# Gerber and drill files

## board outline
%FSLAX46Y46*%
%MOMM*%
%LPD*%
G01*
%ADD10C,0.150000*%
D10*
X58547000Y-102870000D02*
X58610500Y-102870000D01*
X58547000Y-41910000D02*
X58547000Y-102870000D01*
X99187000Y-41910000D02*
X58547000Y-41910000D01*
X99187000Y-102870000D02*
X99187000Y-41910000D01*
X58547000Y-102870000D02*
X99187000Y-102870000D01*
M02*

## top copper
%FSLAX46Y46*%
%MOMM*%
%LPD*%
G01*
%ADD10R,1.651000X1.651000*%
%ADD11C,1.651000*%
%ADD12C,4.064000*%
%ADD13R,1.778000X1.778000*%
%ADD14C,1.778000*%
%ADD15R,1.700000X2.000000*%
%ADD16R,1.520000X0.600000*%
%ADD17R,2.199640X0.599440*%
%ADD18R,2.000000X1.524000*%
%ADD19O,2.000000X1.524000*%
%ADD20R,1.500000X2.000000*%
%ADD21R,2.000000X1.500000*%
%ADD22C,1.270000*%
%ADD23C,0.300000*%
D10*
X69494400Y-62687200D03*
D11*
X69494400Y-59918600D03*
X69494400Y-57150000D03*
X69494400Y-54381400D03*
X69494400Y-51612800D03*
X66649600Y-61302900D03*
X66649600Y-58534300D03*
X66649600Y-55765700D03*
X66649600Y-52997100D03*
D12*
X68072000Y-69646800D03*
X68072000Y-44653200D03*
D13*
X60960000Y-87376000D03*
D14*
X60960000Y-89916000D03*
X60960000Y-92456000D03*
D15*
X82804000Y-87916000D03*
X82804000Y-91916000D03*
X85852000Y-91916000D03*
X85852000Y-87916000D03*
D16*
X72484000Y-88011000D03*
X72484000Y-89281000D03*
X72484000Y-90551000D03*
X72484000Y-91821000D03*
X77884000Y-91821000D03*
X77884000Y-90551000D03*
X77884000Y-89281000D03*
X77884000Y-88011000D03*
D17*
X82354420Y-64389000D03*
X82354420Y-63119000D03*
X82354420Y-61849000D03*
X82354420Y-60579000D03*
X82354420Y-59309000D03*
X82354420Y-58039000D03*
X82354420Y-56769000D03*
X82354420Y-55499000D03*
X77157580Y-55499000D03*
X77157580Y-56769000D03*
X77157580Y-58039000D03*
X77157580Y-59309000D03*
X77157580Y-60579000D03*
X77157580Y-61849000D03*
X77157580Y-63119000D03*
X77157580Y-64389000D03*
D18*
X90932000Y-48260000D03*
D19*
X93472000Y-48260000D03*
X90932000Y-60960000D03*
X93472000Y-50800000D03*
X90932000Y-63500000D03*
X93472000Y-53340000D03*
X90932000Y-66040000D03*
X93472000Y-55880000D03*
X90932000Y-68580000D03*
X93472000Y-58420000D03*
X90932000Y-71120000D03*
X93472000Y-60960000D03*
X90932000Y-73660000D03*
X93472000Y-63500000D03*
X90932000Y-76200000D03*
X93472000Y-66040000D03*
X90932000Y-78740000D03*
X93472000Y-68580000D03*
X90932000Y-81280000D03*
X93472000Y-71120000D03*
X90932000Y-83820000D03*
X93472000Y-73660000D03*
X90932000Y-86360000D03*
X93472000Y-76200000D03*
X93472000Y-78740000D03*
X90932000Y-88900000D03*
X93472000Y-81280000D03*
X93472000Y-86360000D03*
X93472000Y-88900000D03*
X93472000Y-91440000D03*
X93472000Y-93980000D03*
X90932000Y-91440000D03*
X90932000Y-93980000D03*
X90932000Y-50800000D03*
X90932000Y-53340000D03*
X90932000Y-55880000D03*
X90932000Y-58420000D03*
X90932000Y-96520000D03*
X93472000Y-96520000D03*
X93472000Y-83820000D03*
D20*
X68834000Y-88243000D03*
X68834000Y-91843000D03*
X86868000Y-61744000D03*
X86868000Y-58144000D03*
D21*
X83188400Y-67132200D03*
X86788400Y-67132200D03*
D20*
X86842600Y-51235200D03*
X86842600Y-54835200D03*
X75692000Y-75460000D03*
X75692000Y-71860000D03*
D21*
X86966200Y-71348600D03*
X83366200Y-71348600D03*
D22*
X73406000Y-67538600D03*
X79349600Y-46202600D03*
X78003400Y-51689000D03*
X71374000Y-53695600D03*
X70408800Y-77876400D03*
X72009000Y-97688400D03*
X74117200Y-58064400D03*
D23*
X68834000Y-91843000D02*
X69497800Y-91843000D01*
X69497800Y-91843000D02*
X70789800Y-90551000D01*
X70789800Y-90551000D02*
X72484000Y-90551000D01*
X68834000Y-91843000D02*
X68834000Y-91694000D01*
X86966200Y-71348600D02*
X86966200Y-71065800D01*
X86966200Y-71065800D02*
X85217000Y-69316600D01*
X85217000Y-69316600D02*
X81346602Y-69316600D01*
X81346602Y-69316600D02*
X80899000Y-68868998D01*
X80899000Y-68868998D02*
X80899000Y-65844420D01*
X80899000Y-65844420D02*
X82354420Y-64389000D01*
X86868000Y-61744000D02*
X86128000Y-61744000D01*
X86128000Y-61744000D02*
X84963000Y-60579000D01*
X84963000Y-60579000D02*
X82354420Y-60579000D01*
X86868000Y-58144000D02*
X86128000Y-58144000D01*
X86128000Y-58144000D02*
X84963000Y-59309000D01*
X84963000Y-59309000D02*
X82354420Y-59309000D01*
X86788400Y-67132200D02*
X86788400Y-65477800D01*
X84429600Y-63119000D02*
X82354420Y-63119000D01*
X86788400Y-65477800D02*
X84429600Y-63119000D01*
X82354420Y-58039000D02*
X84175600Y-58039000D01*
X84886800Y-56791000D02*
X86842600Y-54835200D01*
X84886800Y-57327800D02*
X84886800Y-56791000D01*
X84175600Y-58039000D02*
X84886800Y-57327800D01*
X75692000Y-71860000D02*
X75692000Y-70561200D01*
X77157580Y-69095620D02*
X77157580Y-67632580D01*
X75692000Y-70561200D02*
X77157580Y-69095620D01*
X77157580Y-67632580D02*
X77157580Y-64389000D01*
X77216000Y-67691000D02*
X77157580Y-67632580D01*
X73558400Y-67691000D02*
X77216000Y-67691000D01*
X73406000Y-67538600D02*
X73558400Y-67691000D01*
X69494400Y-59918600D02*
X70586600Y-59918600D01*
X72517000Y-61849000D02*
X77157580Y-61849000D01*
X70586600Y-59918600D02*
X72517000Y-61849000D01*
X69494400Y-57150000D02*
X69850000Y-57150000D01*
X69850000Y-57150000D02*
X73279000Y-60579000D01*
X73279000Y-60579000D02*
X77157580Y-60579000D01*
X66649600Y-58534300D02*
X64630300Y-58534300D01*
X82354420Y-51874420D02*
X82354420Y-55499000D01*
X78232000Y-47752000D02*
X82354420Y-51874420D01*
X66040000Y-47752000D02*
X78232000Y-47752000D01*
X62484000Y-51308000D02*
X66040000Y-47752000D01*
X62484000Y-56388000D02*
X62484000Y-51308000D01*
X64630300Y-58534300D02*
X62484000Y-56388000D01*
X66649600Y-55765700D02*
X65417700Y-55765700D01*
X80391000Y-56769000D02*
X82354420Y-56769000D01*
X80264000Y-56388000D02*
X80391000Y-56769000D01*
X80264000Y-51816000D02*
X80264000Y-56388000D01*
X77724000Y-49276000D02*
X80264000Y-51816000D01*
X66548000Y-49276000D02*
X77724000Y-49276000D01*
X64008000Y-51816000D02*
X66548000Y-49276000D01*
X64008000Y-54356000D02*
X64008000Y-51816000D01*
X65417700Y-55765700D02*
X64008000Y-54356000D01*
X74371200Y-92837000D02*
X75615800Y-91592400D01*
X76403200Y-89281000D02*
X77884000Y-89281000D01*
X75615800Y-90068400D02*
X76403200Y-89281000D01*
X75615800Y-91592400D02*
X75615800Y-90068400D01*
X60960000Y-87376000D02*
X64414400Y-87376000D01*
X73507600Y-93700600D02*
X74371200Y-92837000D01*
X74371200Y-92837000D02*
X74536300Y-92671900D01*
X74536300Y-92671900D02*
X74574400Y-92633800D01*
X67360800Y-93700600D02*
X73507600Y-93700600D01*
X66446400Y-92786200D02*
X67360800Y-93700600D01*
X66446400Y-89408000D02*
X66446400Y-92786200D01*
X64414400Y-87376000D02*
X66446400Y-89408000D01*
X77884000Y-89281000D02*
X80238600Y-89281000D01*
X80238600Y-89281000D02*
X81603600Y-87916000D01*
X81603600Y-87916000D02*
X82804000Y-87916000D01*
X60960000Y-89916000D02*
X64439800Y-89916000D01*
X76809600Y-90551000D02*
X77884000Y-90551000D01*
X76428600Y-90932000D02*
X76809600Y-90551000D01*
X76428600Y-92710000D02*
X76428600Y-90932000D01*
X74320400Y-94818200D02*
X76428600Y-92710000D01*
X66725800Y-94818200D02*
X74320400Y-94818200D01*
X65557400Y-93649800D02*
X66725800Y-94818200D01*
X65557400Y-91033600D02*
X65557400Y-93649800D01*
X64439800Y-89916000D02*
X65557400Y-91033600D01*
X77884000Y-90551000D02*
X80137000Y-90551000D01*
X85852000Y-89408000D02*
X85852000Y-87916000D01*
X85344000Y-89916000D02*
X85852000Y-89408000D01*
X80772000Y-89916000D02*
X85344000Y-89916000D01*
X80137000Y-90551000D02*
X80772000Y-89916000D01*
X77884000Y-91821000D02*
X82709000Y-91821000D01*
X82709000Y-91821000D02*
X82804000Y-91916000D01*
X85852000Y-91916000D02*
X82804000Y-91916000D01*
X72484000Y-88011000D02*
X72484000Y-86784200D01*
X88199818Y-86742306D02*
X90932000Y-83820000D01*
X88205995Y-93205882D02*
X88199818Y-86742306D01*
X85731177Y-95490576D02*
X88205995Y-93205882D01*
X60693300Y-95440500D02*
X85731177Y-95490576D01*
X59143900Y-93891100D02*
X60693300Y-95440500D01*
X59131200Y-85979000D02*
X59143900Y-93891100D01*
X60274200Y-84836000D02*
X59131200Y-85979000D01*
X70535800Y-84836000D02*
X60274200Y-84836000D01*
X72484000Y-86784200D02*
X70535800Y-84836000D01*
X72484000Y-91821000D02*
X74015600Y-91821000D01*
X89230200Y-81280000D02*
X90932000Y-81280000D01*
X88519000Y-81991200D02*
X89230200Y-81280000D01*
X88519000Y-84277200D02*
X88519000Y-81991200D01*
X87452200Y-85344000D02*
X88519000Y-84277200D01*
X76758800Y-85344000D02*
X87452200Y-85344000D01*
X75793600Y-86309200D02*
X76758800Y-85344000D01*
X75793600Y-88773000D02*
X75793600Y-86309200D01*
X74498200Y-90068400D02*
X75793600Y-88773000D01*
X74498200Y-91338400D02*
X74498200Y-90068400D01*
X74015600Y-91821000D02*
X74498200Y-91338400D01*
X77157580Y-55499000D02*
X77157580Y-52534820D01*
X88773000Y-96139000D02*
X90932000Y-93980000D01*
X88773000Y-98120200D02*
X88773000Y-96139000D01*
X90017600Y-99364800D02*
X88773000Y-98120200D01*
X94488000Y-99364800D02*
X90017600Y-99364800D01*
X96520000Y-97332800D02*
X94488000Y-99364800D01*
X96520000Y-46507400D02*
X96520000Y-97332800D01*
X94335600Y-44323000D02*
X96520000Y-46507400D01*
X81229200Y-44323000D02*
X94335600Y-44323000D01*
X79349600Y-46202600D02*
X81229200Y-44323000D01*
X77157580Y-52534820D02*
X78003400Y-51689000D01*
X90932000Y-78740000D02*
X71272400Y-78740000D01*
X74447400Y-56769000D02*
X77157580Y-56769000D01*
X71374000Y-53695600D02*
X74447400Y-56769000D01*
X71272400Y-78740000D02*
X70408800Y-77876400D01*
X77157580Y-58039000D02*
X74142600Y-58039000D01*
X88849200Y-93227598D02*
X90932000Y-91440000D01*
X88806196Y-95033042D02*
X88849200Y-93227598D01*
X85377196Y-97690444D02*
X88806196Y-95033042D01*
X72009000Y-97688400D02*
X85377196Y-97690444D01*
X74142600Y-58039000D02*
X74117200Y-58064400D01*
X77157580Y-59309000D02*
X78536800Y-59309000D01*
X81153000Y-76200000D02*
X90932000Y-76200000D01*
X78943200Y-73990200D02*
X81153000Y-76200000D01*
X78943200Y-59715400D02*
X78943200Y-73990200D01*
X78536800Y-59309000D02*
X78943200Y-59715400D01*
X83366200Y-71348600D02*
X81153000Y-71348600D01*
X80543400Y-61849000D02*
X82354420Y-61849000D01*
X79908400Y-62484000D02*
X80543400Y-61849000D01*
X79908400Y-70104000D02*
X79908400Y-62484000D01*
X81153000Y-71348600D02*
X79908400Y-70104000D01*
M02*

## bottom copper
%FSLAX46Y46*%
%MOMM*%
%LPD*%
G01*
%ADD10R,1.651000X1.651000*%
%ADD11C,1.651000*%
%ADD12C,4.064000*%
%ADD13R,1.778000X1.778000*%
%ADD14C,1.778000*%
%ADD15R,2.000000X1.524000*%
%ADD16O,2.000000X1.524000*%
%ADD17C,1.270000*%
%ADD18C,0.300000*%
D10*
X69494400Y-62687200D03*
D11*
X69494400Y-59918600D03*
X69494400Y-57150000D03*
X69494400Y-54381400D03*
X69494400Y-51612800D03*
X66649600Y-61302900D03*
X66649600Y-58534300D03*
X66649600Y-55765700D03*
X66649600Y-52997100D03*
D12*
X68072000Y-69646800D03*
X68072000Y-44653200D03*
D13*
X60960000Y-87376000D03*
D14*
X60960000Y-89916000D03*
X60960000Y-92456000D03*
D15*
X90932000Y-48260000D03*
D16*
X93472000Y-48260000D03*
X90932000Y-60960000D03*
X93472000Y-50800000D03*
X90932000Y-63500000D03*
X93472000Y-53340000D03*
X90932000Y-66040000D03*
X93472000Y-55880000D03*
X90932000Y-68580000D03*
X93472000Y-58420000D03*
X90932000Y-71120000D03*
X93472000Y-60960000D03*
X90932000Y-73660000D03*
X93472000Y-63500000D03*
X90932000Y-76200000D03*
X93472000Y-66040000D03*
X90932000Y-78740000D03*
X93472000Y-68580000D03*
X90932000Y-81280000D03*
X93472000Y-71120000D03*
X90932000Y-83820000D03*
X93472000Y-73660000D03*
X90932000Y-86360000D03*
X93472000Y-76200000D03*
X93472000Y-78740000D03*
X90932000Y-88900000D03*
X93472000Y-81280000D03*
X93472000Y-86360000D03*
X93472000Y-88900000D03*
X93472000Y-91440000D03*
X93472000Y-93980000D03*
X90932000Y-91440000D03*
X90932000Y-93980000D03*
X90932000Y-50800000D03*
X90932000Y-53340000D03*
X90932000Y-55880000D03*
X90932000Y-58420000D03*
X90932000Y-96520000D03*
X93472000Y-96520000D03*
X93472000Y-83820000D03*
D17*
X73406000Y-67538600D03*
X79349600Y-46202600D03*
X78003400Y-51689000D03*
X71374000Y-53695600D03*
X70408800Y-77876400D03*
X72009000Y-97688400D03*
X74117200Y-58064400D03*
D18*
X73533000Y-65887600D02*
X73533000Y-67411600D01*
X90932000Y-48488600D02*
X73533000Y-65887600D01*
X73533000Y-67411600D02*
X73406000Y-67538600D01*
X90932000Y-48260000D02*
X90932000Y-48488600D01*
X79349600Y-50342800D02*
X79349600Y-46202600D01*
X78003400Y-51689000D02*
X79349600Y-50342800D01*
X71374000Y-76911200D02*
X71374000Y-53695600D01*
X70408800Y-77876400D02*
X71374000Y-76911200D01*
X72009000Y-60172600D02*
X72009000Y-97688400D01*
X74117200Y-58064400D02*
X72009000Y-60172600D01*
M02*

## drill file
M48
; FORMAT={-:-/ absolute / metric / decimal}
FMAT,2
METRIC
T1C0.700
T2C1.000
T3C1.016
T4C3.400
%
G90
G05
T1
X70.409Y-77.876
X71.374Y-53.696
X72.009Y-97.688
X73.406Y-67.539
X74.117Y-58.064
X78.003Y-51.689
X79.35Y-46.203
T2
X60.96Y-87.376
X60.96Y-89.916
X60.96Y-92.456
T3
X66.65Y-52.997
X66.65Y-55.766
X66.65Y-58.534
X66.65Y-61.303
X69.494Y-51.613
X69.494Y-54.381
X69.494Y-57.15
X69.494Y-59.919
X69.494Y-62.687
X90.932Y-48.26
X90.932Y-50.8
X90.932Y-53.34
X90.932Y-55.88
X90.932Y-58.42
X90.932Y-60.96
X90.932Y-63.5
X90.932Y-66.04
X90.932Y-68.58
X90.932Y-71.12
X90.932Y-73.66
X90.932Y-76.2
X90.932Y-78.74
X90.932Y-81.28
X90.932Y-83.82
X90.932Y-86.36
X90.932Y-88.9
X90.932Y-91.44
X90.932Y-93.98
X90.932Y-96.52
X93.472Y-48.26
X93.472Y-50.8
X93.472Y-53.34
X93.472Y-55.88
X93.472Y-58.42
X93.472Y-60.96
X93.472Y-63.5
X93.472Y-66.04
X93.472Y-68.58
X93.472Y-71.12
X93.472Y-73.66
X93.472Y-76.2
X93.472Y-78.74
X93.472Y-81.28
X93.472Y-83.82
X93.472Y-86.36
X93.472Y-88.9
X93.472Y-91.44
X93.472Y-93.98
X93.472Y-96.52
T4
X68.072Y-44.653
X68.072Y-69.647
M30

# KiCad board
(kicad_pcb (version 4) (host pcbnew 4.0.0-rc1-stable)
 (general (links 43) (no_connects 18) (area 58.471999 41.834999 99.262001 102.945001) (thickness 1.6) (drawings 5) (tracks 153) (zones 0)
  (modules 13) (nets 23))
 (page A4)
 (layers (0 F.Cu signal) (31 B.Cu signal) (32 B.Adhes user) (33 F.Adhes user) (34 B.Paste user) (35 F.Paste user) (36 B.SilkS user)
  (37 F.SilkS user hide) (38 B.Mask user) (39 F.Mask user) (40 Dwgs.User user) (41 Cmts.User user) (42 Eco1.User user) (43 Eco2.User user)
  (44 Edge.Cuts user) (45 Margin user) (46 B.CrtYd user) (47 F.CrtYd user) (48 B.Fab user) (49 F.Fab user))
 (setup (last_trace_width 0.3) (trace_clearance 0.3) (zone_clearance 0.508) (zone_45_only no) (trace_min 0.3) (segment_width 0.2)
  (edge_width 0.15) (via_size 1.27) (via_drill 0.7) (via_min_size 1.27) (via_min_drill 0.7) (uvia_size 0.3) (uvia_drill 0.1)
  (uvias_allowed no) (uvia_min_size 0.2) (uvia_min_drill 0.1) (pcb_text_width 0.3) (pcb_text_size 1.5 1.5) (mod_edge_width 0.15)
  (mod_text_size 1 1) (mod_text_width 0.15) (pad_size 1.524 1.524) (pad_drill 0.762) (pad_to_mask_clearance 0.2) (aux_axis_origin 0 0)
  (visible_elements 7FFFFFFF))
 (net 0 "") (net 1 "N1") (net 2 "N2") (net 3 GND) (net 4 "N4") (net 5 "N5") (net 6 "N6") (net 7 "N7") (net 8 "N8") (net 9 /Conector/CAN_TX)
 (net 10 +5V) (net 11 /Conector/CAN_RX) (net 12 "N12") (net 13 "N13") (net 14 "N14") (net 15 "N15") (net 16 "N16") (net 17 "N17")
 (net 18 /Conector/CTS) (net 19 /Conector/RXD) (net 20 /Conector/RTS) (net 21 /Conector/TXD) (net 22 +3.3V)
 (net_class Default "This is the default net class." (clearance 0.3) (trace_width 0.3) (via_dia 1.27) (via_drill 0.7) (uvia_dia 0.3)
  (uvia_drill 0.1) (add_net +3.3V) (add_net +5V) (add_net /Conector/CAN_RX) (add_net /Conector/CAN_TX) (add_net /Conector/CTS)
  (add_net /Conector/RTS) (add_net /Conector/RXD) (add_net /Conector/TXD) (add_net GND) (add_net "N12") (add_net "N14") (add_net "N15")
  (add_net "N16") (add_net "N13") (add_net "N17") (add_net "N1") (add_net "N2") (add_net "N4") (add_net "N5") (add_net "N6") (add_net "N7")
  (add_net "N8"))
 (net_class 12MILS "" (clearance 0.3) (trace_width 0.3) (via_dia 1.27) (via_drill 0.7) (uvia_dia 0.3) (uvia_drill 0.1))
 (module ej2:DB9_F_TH (layer F.Cu) (at 68.072 57.15 90)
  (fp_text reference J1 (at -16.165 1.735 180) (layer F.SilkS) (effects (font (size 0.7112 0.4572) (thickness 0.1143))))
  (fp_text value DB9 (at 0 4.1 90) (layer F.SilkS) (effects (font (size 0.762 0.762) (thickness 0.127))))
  (pad 1 thru_hole rect (at -5.5372 1.4224 90) (size 1.651 1.651) (drill 1.016) (layers *.Cu *.Mask))
  (pad 2 thru_hole circle (at -2.7686 1.4224 90) (size 1.651 1.651) (drill 1.016) (layers *.Cu *.Mask) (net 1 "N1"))
  (pad 3 thru_hole circle (at 0 1.4224 90) (size 1.651 1.651) (drill 1.016) (layers *.Cu *.Mask) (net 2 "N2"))
  (pad 4 thru_hole circle (at 2.7686 1.4224 90) (size 1.651 1.651) (drill 1.016) (layers *.Cu *.Mask))
  (pad 5 thru_hole circle (at 5.5372 1.4224 90) (size 1.651 1.651) (drill 1.016) (layers *.Cu *.Mask) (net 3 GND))
  (pad 6 thru_hole circle (at -4.1529 -1.4224 90) (size 1.651 1.651) (drill 1.016) (layers *.Cu *.Mask))
  (pad 7 thru_hole circle (at -1.3843 -1.4224 90) (size 1.651 1.651) (drill 1.016) (layers *.Cu *.Mask) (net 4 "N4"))
  (pad 8 thru_hole circle (at 1.3843 -1.4224 90) (size 1.651 1.651) (drill 1.016) (layers *.Cu *.Mask) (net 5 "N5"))
  (pad 9 thru_hole circle (at 4.1529 -1.4224 90) (size 1.651 1.651) (drill 1.016) (layers *.Cu *.Mask))
  (pad 10 thru_hole circle (at -12.4968 0 90) (size 4.064 4.064) (drill 3.4) (layers *.Cu *.Mask))
  (pad 11 thru_hole circle (at 12.4968 0 90) (size 4.064 4.064) (drill 3.4) (layers *.Cu *.Mask)))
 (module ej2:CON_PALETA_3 (layer F.Cu) (at 60.96 89.916 270)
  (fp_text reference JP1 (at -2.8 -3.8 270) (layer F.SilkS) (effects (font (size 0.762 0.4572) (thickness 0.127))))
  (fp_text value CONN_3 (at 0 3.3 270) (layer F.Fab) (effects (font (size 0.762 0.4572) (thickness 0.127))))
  (pad 1 thru_hole rect (at -2.54 0 270) (size 1.778 1.778) (drill 1) (layers *.Cu *.Mask) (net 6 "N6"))
  (pad 2 thru_hole circle (at 0 0 270) (size 1.778 1.778) (drill 1) (layers *.Cu *.Mask) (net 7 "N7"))
  (pad 3 thru_hole circle (at 2.54 0 270) (size 1.778 1.778) (drill 1) (layers *.Cu *.Mask)))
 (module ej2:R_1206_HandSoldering (layer F.Cu) (at 82.804 89.916 270)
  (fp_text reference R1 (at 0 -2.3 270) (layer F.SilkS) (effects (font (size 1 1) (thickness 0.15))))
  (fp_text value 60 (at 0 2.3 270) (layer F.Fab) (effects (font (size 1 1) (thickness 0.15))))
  (pad 1 smd rect (at -2 0 270) (size 2 1.7) (layers F.Cu F.Paste F.Mask) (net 6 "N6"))
  (pad 2 smd rect (at 2 0 270) (size 2 1.7) (layers F.Cu F.Paste F.Mask) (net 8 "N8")))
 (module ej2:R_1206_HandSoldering (layer F.Cu) (at 85.852 89.916 90)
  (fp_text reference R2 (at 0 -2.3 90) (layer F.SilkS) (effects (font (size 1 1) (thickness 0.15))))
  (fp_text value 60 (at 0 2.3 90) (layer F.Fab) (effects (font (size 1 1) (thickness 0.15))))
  (pad 1 smd rect (at -2 0 90) (size 2 1.7) (layers F.Cu F.Paste F.Mask) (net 8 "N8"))
  (pad 2 smd rect (at 2 0 90) (size 2 1.7) (layers F.Cu F.Paste F.Mask) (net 7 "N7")))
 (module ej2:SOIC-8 (layer F.Cu) (at 75.184 89.916)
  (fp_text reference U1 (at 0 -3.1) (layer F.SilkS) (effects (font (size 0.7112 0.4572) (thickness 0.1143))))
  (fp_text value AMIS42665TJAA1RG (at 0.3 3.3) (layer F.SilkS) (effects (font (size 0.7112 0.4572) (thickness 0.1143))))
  (pad 1 smd rect (at -2.7 -1.905 270) (size 0.6 1.52) (layers F.Cu F.Paste F.Mask) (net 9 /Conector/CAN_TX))
  (pad 2 smd rect (at -2.7 -0.635 270) (size 0.6 1.52) (layers F.Cu F.Paste F.Mask) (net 3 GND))
  (pad 3 smd rect (at -2.7 0.635 270) (size 0.6 1.52) (layers F.Cu F.Paste F.Mask) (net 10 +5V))
  (pad 4 smd rect (at -2.7 1.905 270) (size 0.6 1.52) (layers F.Cu F.Paste F.Mask) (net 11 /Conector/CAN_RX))
  (pad 5 smd rect (at 2.7 1.905 270) (size 0.6 1.52) (layers F.Cu F.Paste F.Mask) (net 8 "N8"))
  (pad 6 smd rect (at 2.7 0.635 270) (size 0.6 1.52) (layers F.Cu F.Paste F.Mask) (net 7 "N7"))
  (pad 7 smd rect (at 2.7 -0.635 270) (size 0.6 1.52) (layers F.Cu F.Paste F.Mask) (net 6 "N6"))
  (pad 8 smd rect (at 2.7 -1.905 270) (size 0.6 1.52) (layers F.Cu F.Paste F.Mask) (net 3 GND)))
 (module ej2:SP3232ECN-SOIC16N (layer F.Cu) (at 79.756 59.944 90)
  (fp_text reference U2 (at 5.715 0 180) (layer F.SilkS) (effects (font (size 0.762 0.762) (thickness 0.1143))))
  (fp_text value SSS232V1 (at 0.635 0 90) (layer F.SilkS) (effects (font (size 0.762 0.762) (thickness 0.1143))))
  (pad 1 smd rect (at -4.445 2.59842 90) (size 0.59944 2.19964) (layers F.Cu F.Paste F.Mask) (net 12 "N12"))
  (pad 2 smd rect (at -3.175 2.59842 90) (size 0.59944 2.19964) (layers F.Cu F.Paste F.Mask) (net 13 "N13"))
  (pad 3 smd rect (at -1.905 2.59842 90) (size 0.59944 2.19964) (layers F.Cu F.Paste F.Mask) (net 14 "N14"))
  (pad 4 smd rect (at -0.635 2.59842 90) (size 0.59944 2.19964) (layers F.Cu F.Paste F.Mask) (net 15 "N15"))
  (pad 5 smd rect (at 0.635 2.59842 90) (size 0.59944 2.19964) (layers F.Cu F.Paste F.Mask) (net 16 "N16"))
  (pad 6 smd rect (at 1.905 2.59842 90) (size 0.59944 2.19964) (layers F.Cu F.Paste F.Mask) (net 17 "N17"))
  (pad 7 smd rect (at 3.175 2.59842 90) (size 0.59944 2.19964) (layers F.Cu F.Paste F.Mask) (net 5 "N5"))
  (pad 8 smd rect (at 4.445 2.59842 90) (size 0.59944 2.19964) (layers F.Cu F.Paste F.Mask) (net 4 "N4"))
  (pad 9 smd rect (at 4.445 -2.59842 90) (size 0.59944 2.19964) (layers F.Cu F.Paste F.Mask) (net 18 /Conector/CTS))
  (pad 10 smd rect (at 3.175 -2.59842 90) (size 0.59944 2.19964) (layers F.Cu F.Paste F.Mask) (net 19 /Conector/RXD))
  (pad 11 smd rect (at 1.905 -2.59842 90) (size 0.59944 2.19964) (layers F.Cu F.Paste F.Mask) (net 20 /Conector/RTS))
  (pad 12 smd rect (at 0.635 -2.59842 90) (size 0.59944 2.19964) (layers F.Cu F.Paste F.Mask) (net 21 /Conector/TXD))
  (pad 13 smd rect (at -0.635 -2.59842 90) (size 0.59944 2.19964) (layers F.Cu F.Paste F.Mask) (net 2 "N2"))
  (pad 14 smd rect (at -1.905 -2.59842 90) (size 0.59944 2.19964) (layers F.Cu F.Paste F.Mask) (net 1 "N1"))
  (pad 15 smd rect (at -3.175 -2.59842 90) (size 0.59944 2.19964) (layers F.Cu F.Paste F.Mask) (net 3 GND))
  (pad 16 smd rect (at -4.445 -2.59842 90) (size 0.59944 2.19964) (layers F.Cu F.Paste F.Mask) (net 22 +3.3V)))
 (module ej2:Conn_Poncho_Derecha (layer F.Cu) (at 90.932 48.26)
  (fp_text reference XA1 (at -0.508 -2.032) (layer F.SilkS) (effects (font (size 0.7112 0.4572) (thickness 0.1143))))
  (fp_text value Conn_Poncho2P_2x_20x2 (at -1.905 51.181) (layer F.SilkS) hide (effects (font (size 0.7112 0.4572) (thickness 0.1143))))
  (pad 1 thru_hole rect (at 0 0 270) (size 1.524 2) (drill 1.016) (layers *.Cu *.Mask) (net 22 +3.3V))
  (pad 2 thru_hole oval (at 2.54 0 270) (size 1.524 2) (drill 1.016) (layers *.Cu *.Mask) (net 10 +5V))
  (pad 11 thru_hole oval (at 0 12.7 270) (size 1.524 2) (drill 1.016) (layers *.Cu *.Mask))
  (pad 4 thru_hole oval (at 2.54 2.54 270) (size 1.524 2) (drill 1.016) (layers *.Cu *.Mask) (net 3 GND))
  (pad 13 thru_hole oval (at 0 15.24 270) (size 1.524 2) (drill 1.016) (layers *.Cu *.Mask))
  (pad 6 thru_hole oval (at 2.54 5.08 270) (size 1.524 2) (drill 1.016) (layers *.Cu *.Mask))
  (pad 15 thru_hole oval (at 0 17.78 270) (size 1.524 2) (drill 1.016) (layers *.Cu *.Mask))
  (pad 8 thru_hole oval (at 2.54 7.62 270) (size 1.524 2) (drill 1.016) (layers *.Cu *.Mask))
  (pad 17 thru_hole oval (at 0 20.32 270) (size 1.524 2) (drill 1.016) (layers *.Cu *.Mask))
  (pad 10 thru_hole oval (at 2.54 10.16 270) (size 1.524 2) (drill 1.016) (layers *.Cu *.Mask))
  (pad 19 thru_hole oval (at 0 22.86 270) (size 1.524 2) (drill 1.016) (layers *.Cu *.Mask))
  (pad 12 thru_hole oval (at 2.54 12.7 270) (size 1.524 2) (drill 1.016) (layers *.Cu *.Mask))
  (pad 21 thru_hole oval (at 0 25.4 270) (size 1.524 2) (drill 1.016) (layers *.Cu *.Mask))
  (pad 14 thru_hole oval (at 2.54 15.24 270) (size 1.524 2) (drill 1.016) (layers *.Cu *.Mask))
  (pad 23 thru_hole oval (at 0 27.94 270) (size 1.524 2) (drill 1.016) (layers *.Cu *.Mask) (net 21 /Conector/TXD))
  (pad 16 thru_hole oval (at 2.54 17.78 270) (size 1.524 2) (drill 1.016) (layers *.Cu *.Mask))
  (pad 25 thru_hole oval (at 0 30.48 270) (size 1.524 2) (drill 1.016) (layers *.Cu *.Mask) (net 19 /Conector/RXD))
  (pad 18 thru_hole oval (at 2.54 20.32 270) (size 1.524 2) (drill 1.016) (layers *.Cu *.Mask))
  (pad 27 thru_hole oval (at 0 33.02 270) (size 1.524 2) (drill 1.016) (layers *.Cu *.Mask) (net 11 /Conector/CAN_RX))
  (pad 20 thru_hole oval (at 2.54 22.86 270) (size 1.524 2) (drill 1.016) (layers *.Cu *.Mask) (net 3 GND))
  (pad 29 thru_hole oval (at 0 35.56 270) (size 1.524 2) (drill 1.016) (layers *.Cu *.Mask) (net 9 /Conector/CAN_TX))
  (pad 22 thru_hole oval (at 2.54 25.4 270) (size 1.524 2) (drill 1.016) (layers *.Cu *.Mask) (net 3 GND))
  (pad 31 thru_hole oval (at 0 38.1 270) (size 1.524 2) (drill 1.016) (layers *.Cu *.Mask))
  (pad 24 thru_hole oval (at 2.54 27.94 270) (size 1.524 2) (drill 1.016) (layers *.Cu *.Mask) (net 3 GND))
  (pad 26 thru_hole oval (at 2.54 30.48 270) (size 1.524 2) (drill 1.016) (layers *.Cu *.Mask) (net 3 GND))
  (pad 33 thru_hole oval (at 0 40.64 270) (size 1.524 2) (drill 1.016) (layers *.Cu *.Mask))
  (pad 28 thru_hole oval (at 2.54 33.02 270) (size 1.524 2) (drill 1.016) (layers *.Cu *.Mask) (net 3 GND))
  (pad 32 thru_hole oval (at 2.54 38.1 270) (size 1.524 2) (drill 1.016) (layers *.Cu *.Mask) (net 3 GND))
  (pad 34 thru_hole oval (at 2.54 40.64 270) (size 1.524 2) (drill 1.016) (layers *.Cu *.Mask))
  (pad 36 thru_hole oval (at 2.54 43.18 270) (size 1.524 2) (drill 1.016) (layers *.Cu *.Mask))
  (pad 38 thru_hole oval (at 2.54 45.72 270) (size 1.524 2) (drill 1.016) (layers *.Cu *.Mask) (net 3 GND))
  (pad 35 thru_hole oval (at 0 43.18 270) (size 1.524 2) (drill 1.016) (layers *.Cu *.Mask) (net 20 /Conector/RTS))
  (pad 37 thru_hole oval (at 0 45.72 270) (size 1.524 2) (drill 1.016) (layers *.Cu *.Mask) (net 18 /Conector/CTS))
  (pad 3 thru_hole oval (at 0 2.54 270) (size 1.524 2) (drill 1.016) (layers *.Cu *.Mask))
  (pad 5 thru_hole oval (at 0 5.08 270) (size 1.524 2) (drill 1.016) (layers *.Cu *.Mask))
  (pad 7 thru_hole oval (at 0 7.62 270) (size 1.524 2) (drill 1.016) (layers *.Cu *.Mask))
  (pad 9 thru_hole oval (at 0 10.16 270) (size 1.524 2) (drill 1.016) (layers *.Cu *.Mask))
  (pad 39 thru_hole oval (at 0 48.26 270) (size 1.524 2) (drill 1.016) (layers *.Cu *.Mask))
  (pad 40 thru_hole oval (at 2.54 48.26 270) (size 1.524 2) (drill 1.016) (layers *.Cu *.Mask) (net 3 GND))
  (pad 30 thru_hole oval (at 2.54 35.56 270) (size 1.524 2) (drill 1.016) (layers *.Cu *.Mask) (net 3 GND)))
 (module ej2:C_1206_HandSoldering (layer F.Cu) (at 68.834 90.043 270)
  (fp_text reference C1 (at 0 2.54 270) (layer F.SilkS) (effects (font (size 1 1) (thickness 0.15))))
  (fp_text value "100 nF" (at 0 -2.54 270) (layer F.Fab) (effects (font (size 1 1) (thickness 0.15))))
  (pad 1 smd rect (at -1.8 0 270) (size 2 1.5) (layers F.Cu F.Paste F.Mask) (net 3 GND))
  (pad 2 smd rect (at 1.8 0 270) (size 2 1.5) (layers F.Cu F.Paste F.Mask) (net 10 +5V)))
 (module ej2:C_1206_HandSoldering (layer F.Cu) (at 86.868 59.944 90)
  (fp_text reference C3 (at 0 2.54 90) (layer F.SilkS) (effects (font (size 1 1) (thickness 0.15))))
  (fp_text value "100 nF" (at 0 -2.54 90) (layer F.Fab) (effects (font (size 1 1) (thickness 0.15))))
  (pad 1 smd rect (at -1.8 0 90) (size 2 1.5) (layers F.Cu F.Paste F.Mask) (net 15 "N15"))
  (pad 2 smd rect (at 1.8 0 90) (size 2 1.5) (layers F.Cu F.Paste F.Mask) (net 16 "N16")))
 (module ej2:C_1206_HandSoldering (layer F.Cu) (at 84.9884 67.1322)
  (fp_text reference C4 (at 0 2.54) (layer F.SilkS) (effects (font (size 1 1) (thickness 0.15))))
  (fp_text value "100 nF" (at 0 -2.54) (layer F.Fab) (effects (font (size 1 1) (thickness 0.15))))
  (pad 1 smd rect (at -1.8 0) (size 2 1.5) (layers F.Cu F.Paste F.Mask) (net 3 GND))
  (pad 2 smd rect (at 1.8 0) (size 2 1.5) (layers F.Cu F.Paste F.Mask) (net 13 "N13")))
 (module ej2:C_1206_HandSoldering (layer F.Cu) (at 86.8426 53.0352 270)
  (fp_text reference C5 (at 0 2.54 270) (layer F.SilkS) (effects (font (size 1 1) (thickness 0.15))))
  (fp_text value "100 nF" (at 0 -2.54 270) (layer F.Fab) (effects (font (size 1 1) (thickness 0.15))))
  (pad 1 smd rect (at -1.8 0 270) (size 2 1.5) (layers F.Cu F.Paste F.Mask) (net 3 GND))
  (pad 2 smd rect (at 1.8 0 270) (size 2 1.5) (layers F.Cu F.Paste F.Mask) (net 17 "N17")))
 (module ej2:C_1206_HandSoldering (layer F.Cu) (at 75.692 73.66 90)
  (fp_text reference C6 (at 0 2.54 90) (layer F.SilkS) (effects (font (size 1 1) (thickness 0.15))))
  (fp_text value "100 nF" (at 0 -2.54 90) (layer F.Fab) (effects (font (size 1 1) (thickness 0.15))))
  (pad 1 smd rect (at -1.8 0 90) (size 2 1.5) (layers F.Cu F.Paste F.Mask) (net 3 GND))
  (pad 2 smd rect (at 1.8 0 90) (size 2 1.5) (layers F.Cu F.Paste F.Mask) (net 22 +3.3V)))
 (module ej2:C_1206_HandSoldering (layer F.Cu) (at 85.1662 71.3486 180)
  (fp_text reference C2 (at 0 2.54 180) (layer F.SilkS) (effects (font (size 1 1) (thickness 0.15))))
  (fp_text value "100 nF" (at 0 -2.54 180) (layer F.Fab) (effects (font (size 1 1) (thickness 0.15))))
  (pad 1 smd rect (at -1.8 0 180) (size 2 1.5) (layers F.Cu F.Paste F.Mask) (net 12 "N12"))
  (pad 2 smd rect (at 1.8 0 180) (size 2 1.5) (layers F.Cu F.Paste F.Mask) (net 14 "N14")))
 (gr_line (start 58.547 102.87) (end 58.6105 102.87) (angle 90) (layer Edge.Cuts) (width 0.15))
 (gr_line (start 58.547 41.91) (end 58.547 102.87) (angle 90) (layer Edge.Cuts) (width 0.15))
 (gr_line (start 99.187 41.91) (end 58.547 41.91) (angle 90) (layer Edge.Cuts) (width 0.15))
 (gr_line (start 99.187 102.87) (end 99.187 41.91) (angle 90) (layer Edge.Cuts) (width 0.15))
 (gr_line (start 58.547 102.87) (end 99.187 102.87) (angle 90) (layer Edge.Cuts) (width 0.15))
 (segment (start 68.834 91.843) (end 69.4978 91.843) (width 0.3) (layer F.Cu) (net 10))
 (segment (start 69.4978 91.843) (end 70.7898 90.551) (width 0.3) (layer F.Cu) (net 10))
 (segment (start 70.7898 90.551) (end 72.484 90.551) (width 0.3) (layer F.Cu) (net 10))
 (segment (start 68.834 91.843) (end 68.834 91.694) (width 0.3) (layer F.Cu) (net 10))
 (segment (start 86.9662 71.3486) (end 86.9662 71.0658) (width 0.3) (layer F.Cu) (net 12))
 (segment (start 86.9662 71.0658) (end 85.217 69.3166) (width 0.3) (layer F.Cu) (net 12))
 (segment (start 85.217 69.3166) (end 81.346602 69.3166) (width 0.3) (layer F.Cu) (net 12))
 (segment (start 81.346602 69.3166) (end 80.899 68.868998) (width 0.3) (layer F.Cu) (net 12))
 (segment (start 80.899 68.868998) (end 80.899 65.84442) (width 0.3) (layer F.Cu) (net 12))
 (segment (start 80.899 65.84442) (end 82.35442 64.389) (width 0.3) (layer F.Cu) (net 12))
 (segment (start 86.868 61.744) (end 86.128 61.744) (width 0.3) (layer F.Cu) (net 15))
 (segment (start 86.128 61.744) (end 84.963 60.579) (width 0.3) (layer F.Cu) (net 15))
 (segment (start 84.963 60.579) (end 82.35442 60.579) (width 0.3) (layer F.Cu) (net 15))
 (segment (start 86.868 58.144) (end 86.128 58.144) (width 0.3) (layer F.Cu) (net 16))
 (segment (start 86.128 58.144) (end 84.963 59.309) (width 0.3) (layer F.Cu) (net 16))
 (segment (start 84.963 59.309) (end 82.35442 59.309) (width 0.3) (layer F.Cu) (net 16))
 (segment (start 86.7884 67.1322) (end 86.7884 65.4778) (width 0.3) (layer F.Cu) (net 13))
 (segment (start 84.4296 63.119) (end 82.35442 63.119) (width 0.3) (layer F.Cu) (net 13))
 (segment (start 86.7884 65.4778) (end 84.4296 63.119) (width 0.3) (layer F.Cu) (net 13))
 (segment (start 82.35442 58.039) (end 84.1756 58.039) (width 0.3) (layer F.Cu) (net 17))
 (segment (start 84.8868 56.791) (end 86.8426 54.8352) (width 0.3) (layer F.Cu) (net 17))
 (segment (start 84.8868 57.3278) (end 84.8868 56.791) (width 0.3) (layer F.Cu) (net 17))
 (segment (start 84.1756 58.039) (end 84.8868 57.3278) (width 0.3) (layer F.Cu) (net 17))
 (segment (start 75.692 71.86) (end 75.692 70.5612) (width 0.3) (layer F.Cu) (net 22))
 (segment (start 77.15758 69.09562) (end 77.15758 67.63258) (width 0.3) (layer F.Cu) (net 22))
 (segment (start 75.692 70.5612) (end 77.15758 69.09562) (width 0.3) (layer F.Cu) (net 22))
 (segment (start 73.533 65.8876) (end 73.533 67.4116) (width 0.3) (layer B.Cu) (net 22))
 (segment (start 90.932 48.4886) (end 73.533 65.8876) (width 0.3) (layer B.Cu) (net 22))
 (segment (start 77.15758 67.63258) (end 77.15758 64.389) (width 0.3) (layer F.Cu) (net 22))
 (segment (start 77.216 67.691) (end 77.15758 67.63258) (width 0.3) (layer F.Cu) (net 22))
 (segment (start 73.5584 67.691) (end 77.216 67.691) (width 0.3) (layer F.Cu) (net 22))
 (segment (start 73.406 67.5386) (end 73.5584 67.691) (width 0.3) (layer F.Cu) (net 22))
 (via (at 73.406 67.5386) (size 1.27) (drill 0.7) (layers F.Cu B.Cu) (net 22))
 (segment (start 73.533 67.4116) (end 73.406 67.5386) (width 0.3) (layer B.Cu) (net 22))
 (segment (start 90.932 48.26) (end 90.932 48.4886) (width 0.3) (layer B.Cu) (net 22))
 (segment (start 69.4944 59.9186) (end 70.5866 59.9186) (width 0.3) (layer F.Cu) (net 1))
 (segment (start 72.517 61.849) (end 77.15758 61.849) (width 0.3) (layer F.Cu) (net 1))
 (segment (start 70.5866 59.9186) (end 72.517 61.849) (width 0.3) (layer F.Cu) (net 1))
 (segment (start 69.4944 57.15) (end 69.85 57.15) (width 0.3) (layer F.Cu) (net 2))
 (segment (start 69.85 57.15) (end 73.279 60.579) (width 0.3) (layer F.Cu) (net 2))
 (segment (start 73.279 60.579) (end 77.15758 60.579) (width 0.3) (layer F.Cu) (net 2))
 (segment (start 66.6496 58.5343) (end 64.6303 58.5343) (width 0.3) (layer F.Cu) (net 4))
 (segment (start 82.35442 51.87442) (end 82.35442 55.499) (width 0.3) (layer F.Cu) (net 4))
 (segment (start 78.232 47.752) (end 82.35442 51.87442) (width 0.3) (layer F.Cu) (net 4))
 (segment (start 66.04 47.752) (end 78.232 47.752) (width 0.3) (layer F.Cu) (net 4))
 (segment (start 62.484 51.308) (end 66.04 47.752) (width 0.3) (layer F.Cu) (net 4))
 (segment (start 62.484 56.388) (end 62.484 51.308) (width 0.3) (layer F.Cu) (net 4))
 (segment (start 64.6303 58.5343) (end 62.484 56.388) (width 0.3) (layer F.Cu) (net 4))
 (segment (start 66.6496 55.7657) (end 65.4177 55.7657) (width 0.3) (layer F.Cu) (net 5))
 (segment (start 80.391 56.769) (end 82.35442 56.769) (width 0.3) (layer F.Cu) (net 5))
 (segment (start 80.264 56.388) (end 80.391 56.769) (width 0.3) (layer F.Cu) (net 5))
 (segment (start 80.264 51.816) (end 80.264 56.388) (width 0.3) (layer F.Cu) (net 5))
 (segment (start 77.724 49.276) (end 80.264 51.816) (width 0.3) (layer F.Cu) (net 5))
 (segment (start 66.548 49.276) (end 77.724 49.276) (width 0.3) (layer F.Cu) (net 5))
 (segment (start 64.008 51.816) (end 66.548 49.276) (width 0.3) (layer F.Cu) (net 5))
 (segment (start 64.008 54.356) (end 64.008 51.816) (width 0.3) (layer F.Cu) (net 5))
 (segment (start 65.4177 55.7657) (end 64.008 54.356) (width 0.3) (layer F.Cu) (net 5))
 (segment (start 74.3712 92.837) (end 75.6158 91.5924) (width 0.3) (layer F.Cu) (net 6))
 (segment (start 76.4032 89.281) (end 77.884 89.281) (width 0.3) (layer F.Cu) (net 6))
 (segment (start 75.6158 90.0684) (end 76.4032 89.281) (width 0.3) (layer F.Cu) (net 6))
 (segment (start 75.6158 91.5924) (end 75.6158 90.0684) (width 0.3) (layer F.Cu) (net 6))
 (segment (start 60.96 87.376) (end 64.4144 87.376) (width 0.3) (layer F.Cu) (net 6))
 (segment (start 73.5076 93.7006) (end 74.3712 92.837) (width 0.3) (layer F.Cu) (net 6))
 (segment (start 74.3712 92.837) (end 74.5363 92.6719) (width 0.3) (layer F.Cu) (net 6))
 (segment (start 74.5363 92.6719) (end 74.5744 92.6338) (width 0.3) (layer F.Cu) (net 6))
 (segment (start 67.3608 93.7006) (end 73.5076 93.7006) (width 0.3) (layer F.Cu) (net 6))
 (segment (start 66.4464 92.7862) (end 67.3608 93.7006) (width 0.3) (layer F.Cu) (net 6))
 (segment (start 66.4464 89.408) (end 66.4464 92.7862) (width 0.3) (layer F.Cu) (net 6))
 (segment (start 64.4144 87.376) (end 66.4464 89.408) (width 0.3) (layer F.Cu) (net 6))
 (segment (start 77.884 89.281) (end 80.2386 89.281) (width 0.3) (layer F.Cu) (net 6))
 (segment (start 80.2386 89.281) (end 81.6036 87.916) (width 0.3) (layer F.Cu) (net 6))
 (segment (start 81.6036 87.916) (end 82.804 87.916) (width 0.3) (layer F.Cu) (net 6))
 (segment (start 60.96 89.916) (end 64.4398 89.916) (width 0.3) (layer F.Cu) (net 7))
 (segment (start 76.8096 90.551) (end 77.884 90.551) (width 0.3) (layer F.Cu) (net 7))
 (segment (start 76.4286 90.932) (end 76.8096 90.551) (width 0.3) (layer F.Cu) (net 7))
 (segment (start 76.4286 92.71) (end 76.4286 90.932) (width 0.3) (layer F.Cu) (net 7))
 (segment (start 74.3204 94.8182) (end 76.4286 92.71) (width 0.3) (layer F.Cu) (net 7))
 (segment (start 66.7258 94.8182) (end 74.3204 94.8182) (width 0.3) (layer F.Cu) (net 7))
 (segment (start 65.5574 93.6498) (end 66.7258 94.8182) (width 0.3) (layer F.Cu) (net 7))
 (segment (start 65.5574 91.0336) (end 65.5574 93.6498) (width 0.3) (layer F.Cu) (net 7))
 (segment (start 64.4398 89.916) (end 65.5574 91.0336) (width 0.3) (layer F.Cu) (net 7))
 (segment (start 77.884 90.551) (end 80.137 90.551) (width 0.3) (layer F.Cu) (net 7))
 (segment (start 85.852 89.408) (end 85.852 87.916) (width 0.3) (layer F.Cu) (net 7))
 (segment (start 85.344 89.916) (end 85.852 89.408) (width 0.3) (layer F.Cu) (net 7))
 (segment (start 80.772 89.916) (end 85.344 89.916) (width 0.3) (layer F.Cu) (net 7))
 (segment (start 80.137 90.551) (end 80.772 89.916) (width 0.3) (layer F.Cu) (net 7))
 (segment (start 77.884 91.821) (end 82.709 91.821) (width 0.3) (layer F.Cu) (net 8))
 (segment (start 82.709 91.821) (end 82.804 91.916) (width 0.3) (layer F.Cu) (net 8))
 (segment (start 85.852 91.916) (end 82.804 91.916) (width 0.3) (layer F.Cu) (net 8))
 (segment (start 72.484 88.011) (end 72.484 86.7842) (width 0.3) (layer F.Cu) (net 9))
 (segment (start 88.199818 86.742306) (end 90.932 83.82) (width 0.3) (layer F.Cu) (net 9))
 (segment (start 88.205995 93.205882) (end 88.199818 86.742306) (width 0.3) (layer F.Cu) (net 9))
 (segment (start 85.731177 95.490576) (end 88.205995 93.205882) (width 0.3) (layer F.Cu) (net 9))
 (segment (start 60.6933 95.4405) (end 85.731177 95.490576) (width 0.3) (layer F.Cu) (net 9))
 (segment (start 59.1439 93.8911) (end 60.6933 95.4405) (width 0.3) (layer F.Cu) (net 9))
 (segment (start 59.1312 85.979) (end 59.1439 93.8911) (width 0.3) (layer F.Cu) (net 9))
 (segment (start 60.2742 84.836) (end 59.1312 85.979) (width 0.3) (layer F.Cu) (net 9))
 (segment (start 70.5358 84.836) (end 60.2742 84.836) (width 0.3) (layer F.Cu) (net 9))
 (segment (start 72.484 86.7842) (end 70.5358 84.836) (width 0.3) (layer F.Cu) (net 9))
 (segment (start 72.484 91.821) (end 74.0156 91.821) (width 0.3) (layer F.Cu) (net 11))
 (segment (start 89.2302 81.28) (end 90.932 81.28) (width 0.3) (layer F.Cu) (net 11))
 (segment (start 88.519 81.9912) (end 89.2302 81.28) (width 0.3) (layer F.Cu) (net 11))
 (segment (start 88.519 84.2772) (end 88.519 81.9912) (width 0.3) (layer F.Cu) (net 11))
 (segment (start 87.4522 85.344) (end 88.519 84.2772) (width 0.3) (layer F.Cu) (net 11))
 (segment (start 76.7588 85.344) (end 87.4522 85.344) (width 0.3) (layer F.Cu) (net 11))
 (segment (start 75.7936 86.3092) (end 76.7588 85.344) (width 0.3) (layer F.Cu) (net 11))
 (segment (start 75.7936 88.773) (end 75.7936 86.3092) (width 0.3) (layer F.Cu) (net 11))
 (segment (start 74.4982 90.0684) (end 75.7936 88.773) (width 0.3) (layer F.Cu) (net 11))
 (segment (start 74.4982 91.3384) (end 74.4982 90.0684) (width 0.3) (layer F.Cu) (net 11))
 (segment (start 74.0156 91.821) (end 74.4982 91.3384) (width 0.3) (layer F.Cu) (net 11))
 (segment (start 77.15758 55.499) (end 77.15758 52.53482) (width 0.3) (layer F.Cu) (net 18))
 (segment (start 88.773 96.139) (end 90.932 93.98) (width 0.3) (layer F.Cu) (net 18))
 (segment (start 88.773 98.1202) (end 88.773 96.139) (width 0.3) (layer F.Cu) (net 18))
 (segment (start 90.0176 99.3648) (end 88.773 98.1202) (width 0.3) (layer F.Cu) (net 18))
 (segment (start 94.488 99.3648) (end 90.0176 99.3648) (width 0.3) (layer F.Cu) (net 18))
 (segment (start 96.52 97.3328) (end 94.488 99.3648) (width 0.3) (layer F.Cu) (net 18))
 (segment (start 96.52 46.5074) (end 96.52 97.3328) (width 0.3) (layer F.Cu) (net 18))
 (segment (start 94.3356 44.323) (end 96.52 46.5074) (width 0.3) (layer F.Cu) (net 18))
 (segment (start 81.2292 44.323) (end 94.3356 44.323) (width 0.3) (layer F.Cu) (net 18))
 (segment (start 79.3496 46.2026) (end 81.2292 44.323) (width 0.3) (layer F.Cu) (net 18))
 (via (at 79.3496 46.2026) (size 1.27) (drill 0.7) (layers F.Cu B.Cu) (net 18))
 (segment (start 79.3496 50.3428) (end 79.3496 46.2026) (width 0.3) (layer B.Cu) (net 18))
 (segment (start 78.0034 51.689) (end 79.3496 50.3428) (width 0.3) (layer B.Cu) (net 18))
 (via (at 78.0034 51.689) (size 1.27) (drill 0.7) (layers F.Cu B.Cu) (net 18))
 (segment (start 77.15758 52.53482) (end 78.0034 51.689) (width 0.3) (layer F.Cu) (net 18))
 (segment (start 90.932 78.74) (end 71.2724 78.74) (width 0.3) (layer F.Cu) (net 19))
 (segment (start 74.4474 56.769) (end 77.15758 56.769) (width 0.3) (layer F.Cu) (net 19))
 (segment (start 71.374 53.6956) (end 74.4474 56.769) (width 0.3) (layer F.Cu) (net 19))
 (via (at 71.374 53.6956) (size 1.27) (drill 0.7) (layers F.Cu B.Cu) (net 19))
 (segment (start 71.374 76.9112) (end 71.374 53.6956) (width 0.3) (layer B.Cu) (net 19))
 (segment (start 70.4088 77.8764) (end 71.374 76.9112) (width 0.3) (layer B.Cu) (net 19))
 (via (at 70.4088 77.8764) (size 1.27) (drill 0.7) (layers F.Cu B.Cu) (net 19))
 (segment (start 71.2724 78.74) (end 70.4088 77.8764) (width 0.3) (layer F.Cu) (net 19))
 (segment (start 77.15758 58.039) (end 74.1426 58.039) (width 0.3) (layer F.Cu) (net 20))
 (segment (start 88.8492 93.227598) (end 90.932 91.44) (width 0.3) (layer F.Cu) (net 20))
 (segment (start 88.806196 95.033042) (end 88.8492 93.227598) (width 0.3) (layer F.Cu) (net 20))
 (segment (start 85.377196 97.690444) (end 88.806196 95.033042) (width 0.3) (layer F.Cu) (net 20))
 (segment (start 72.009 97.6884) (end 85.377196 97.690444) (width 0.3) (layer F.Cu) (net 20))
 (via (at 72.009 97.6884) (size 1.27) (drill 0.7) (layers F.Cu B.Cu) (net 20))
 (segment (start 72.009 60.1726) (end 72.009 97.6884) (width 0.3) (layer B.Cu) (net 20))
 (segment (start 74.1172 58.0644) (end 72.009 60.1726) (width 0.3) (layer B.Cu) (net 20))
 (via (at 74.1172 58.0644) (size 1.27) (drill 0.7) (layers F.Cu B.Cu) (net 20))
 (segment (start 74.1426 58.039) (end 74.1172 58.0644) (width 0.3) (layer F.Cu) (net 20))
 (segment (start 77.15758 59.309) (end 78.5368 59.309) (width 0.3) (layer F.Cu) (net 21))
 (segment (start 81.153 76.2) (end 90.932 76.2) (width 0.3) (layer F.Cu) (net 21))
 (segment (start 78.9432 73.9902) (end 81.153 76.2) (width 0.3) (layer F.Cu) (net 21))
 (segment (start 78.9432 59.7154) (end 78.9432 73.9902) (width 0.3) (layer F.Cu) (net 21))
 (segment (start 78.5368 59.309) (end 78.9432 59.7154) (width 0.3) (layer F.Cu) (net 21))
 (segment (start 83.3662 71.3486) (end 81.153 71.3486) (width 0.3) (layer F.Cu) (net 14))
 (segment (start 80.5434 61.849) (end 82.35442 61.849) (width 0.3) (layer F.Cu) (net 14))
 (segment (start 79.9084 62.484) (end 80.5434 61.849) (width 0.3) (layer F.Cu) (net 14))
 (segment (start 79.9084 70.104) (end 79.9084 62.484) (width 0.3) (layer F.Cu) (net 14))
 (segment (start 81.153 71.3486) (end 79.9084 70.104) (width 0.3) (layer F.Cu) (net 14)))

